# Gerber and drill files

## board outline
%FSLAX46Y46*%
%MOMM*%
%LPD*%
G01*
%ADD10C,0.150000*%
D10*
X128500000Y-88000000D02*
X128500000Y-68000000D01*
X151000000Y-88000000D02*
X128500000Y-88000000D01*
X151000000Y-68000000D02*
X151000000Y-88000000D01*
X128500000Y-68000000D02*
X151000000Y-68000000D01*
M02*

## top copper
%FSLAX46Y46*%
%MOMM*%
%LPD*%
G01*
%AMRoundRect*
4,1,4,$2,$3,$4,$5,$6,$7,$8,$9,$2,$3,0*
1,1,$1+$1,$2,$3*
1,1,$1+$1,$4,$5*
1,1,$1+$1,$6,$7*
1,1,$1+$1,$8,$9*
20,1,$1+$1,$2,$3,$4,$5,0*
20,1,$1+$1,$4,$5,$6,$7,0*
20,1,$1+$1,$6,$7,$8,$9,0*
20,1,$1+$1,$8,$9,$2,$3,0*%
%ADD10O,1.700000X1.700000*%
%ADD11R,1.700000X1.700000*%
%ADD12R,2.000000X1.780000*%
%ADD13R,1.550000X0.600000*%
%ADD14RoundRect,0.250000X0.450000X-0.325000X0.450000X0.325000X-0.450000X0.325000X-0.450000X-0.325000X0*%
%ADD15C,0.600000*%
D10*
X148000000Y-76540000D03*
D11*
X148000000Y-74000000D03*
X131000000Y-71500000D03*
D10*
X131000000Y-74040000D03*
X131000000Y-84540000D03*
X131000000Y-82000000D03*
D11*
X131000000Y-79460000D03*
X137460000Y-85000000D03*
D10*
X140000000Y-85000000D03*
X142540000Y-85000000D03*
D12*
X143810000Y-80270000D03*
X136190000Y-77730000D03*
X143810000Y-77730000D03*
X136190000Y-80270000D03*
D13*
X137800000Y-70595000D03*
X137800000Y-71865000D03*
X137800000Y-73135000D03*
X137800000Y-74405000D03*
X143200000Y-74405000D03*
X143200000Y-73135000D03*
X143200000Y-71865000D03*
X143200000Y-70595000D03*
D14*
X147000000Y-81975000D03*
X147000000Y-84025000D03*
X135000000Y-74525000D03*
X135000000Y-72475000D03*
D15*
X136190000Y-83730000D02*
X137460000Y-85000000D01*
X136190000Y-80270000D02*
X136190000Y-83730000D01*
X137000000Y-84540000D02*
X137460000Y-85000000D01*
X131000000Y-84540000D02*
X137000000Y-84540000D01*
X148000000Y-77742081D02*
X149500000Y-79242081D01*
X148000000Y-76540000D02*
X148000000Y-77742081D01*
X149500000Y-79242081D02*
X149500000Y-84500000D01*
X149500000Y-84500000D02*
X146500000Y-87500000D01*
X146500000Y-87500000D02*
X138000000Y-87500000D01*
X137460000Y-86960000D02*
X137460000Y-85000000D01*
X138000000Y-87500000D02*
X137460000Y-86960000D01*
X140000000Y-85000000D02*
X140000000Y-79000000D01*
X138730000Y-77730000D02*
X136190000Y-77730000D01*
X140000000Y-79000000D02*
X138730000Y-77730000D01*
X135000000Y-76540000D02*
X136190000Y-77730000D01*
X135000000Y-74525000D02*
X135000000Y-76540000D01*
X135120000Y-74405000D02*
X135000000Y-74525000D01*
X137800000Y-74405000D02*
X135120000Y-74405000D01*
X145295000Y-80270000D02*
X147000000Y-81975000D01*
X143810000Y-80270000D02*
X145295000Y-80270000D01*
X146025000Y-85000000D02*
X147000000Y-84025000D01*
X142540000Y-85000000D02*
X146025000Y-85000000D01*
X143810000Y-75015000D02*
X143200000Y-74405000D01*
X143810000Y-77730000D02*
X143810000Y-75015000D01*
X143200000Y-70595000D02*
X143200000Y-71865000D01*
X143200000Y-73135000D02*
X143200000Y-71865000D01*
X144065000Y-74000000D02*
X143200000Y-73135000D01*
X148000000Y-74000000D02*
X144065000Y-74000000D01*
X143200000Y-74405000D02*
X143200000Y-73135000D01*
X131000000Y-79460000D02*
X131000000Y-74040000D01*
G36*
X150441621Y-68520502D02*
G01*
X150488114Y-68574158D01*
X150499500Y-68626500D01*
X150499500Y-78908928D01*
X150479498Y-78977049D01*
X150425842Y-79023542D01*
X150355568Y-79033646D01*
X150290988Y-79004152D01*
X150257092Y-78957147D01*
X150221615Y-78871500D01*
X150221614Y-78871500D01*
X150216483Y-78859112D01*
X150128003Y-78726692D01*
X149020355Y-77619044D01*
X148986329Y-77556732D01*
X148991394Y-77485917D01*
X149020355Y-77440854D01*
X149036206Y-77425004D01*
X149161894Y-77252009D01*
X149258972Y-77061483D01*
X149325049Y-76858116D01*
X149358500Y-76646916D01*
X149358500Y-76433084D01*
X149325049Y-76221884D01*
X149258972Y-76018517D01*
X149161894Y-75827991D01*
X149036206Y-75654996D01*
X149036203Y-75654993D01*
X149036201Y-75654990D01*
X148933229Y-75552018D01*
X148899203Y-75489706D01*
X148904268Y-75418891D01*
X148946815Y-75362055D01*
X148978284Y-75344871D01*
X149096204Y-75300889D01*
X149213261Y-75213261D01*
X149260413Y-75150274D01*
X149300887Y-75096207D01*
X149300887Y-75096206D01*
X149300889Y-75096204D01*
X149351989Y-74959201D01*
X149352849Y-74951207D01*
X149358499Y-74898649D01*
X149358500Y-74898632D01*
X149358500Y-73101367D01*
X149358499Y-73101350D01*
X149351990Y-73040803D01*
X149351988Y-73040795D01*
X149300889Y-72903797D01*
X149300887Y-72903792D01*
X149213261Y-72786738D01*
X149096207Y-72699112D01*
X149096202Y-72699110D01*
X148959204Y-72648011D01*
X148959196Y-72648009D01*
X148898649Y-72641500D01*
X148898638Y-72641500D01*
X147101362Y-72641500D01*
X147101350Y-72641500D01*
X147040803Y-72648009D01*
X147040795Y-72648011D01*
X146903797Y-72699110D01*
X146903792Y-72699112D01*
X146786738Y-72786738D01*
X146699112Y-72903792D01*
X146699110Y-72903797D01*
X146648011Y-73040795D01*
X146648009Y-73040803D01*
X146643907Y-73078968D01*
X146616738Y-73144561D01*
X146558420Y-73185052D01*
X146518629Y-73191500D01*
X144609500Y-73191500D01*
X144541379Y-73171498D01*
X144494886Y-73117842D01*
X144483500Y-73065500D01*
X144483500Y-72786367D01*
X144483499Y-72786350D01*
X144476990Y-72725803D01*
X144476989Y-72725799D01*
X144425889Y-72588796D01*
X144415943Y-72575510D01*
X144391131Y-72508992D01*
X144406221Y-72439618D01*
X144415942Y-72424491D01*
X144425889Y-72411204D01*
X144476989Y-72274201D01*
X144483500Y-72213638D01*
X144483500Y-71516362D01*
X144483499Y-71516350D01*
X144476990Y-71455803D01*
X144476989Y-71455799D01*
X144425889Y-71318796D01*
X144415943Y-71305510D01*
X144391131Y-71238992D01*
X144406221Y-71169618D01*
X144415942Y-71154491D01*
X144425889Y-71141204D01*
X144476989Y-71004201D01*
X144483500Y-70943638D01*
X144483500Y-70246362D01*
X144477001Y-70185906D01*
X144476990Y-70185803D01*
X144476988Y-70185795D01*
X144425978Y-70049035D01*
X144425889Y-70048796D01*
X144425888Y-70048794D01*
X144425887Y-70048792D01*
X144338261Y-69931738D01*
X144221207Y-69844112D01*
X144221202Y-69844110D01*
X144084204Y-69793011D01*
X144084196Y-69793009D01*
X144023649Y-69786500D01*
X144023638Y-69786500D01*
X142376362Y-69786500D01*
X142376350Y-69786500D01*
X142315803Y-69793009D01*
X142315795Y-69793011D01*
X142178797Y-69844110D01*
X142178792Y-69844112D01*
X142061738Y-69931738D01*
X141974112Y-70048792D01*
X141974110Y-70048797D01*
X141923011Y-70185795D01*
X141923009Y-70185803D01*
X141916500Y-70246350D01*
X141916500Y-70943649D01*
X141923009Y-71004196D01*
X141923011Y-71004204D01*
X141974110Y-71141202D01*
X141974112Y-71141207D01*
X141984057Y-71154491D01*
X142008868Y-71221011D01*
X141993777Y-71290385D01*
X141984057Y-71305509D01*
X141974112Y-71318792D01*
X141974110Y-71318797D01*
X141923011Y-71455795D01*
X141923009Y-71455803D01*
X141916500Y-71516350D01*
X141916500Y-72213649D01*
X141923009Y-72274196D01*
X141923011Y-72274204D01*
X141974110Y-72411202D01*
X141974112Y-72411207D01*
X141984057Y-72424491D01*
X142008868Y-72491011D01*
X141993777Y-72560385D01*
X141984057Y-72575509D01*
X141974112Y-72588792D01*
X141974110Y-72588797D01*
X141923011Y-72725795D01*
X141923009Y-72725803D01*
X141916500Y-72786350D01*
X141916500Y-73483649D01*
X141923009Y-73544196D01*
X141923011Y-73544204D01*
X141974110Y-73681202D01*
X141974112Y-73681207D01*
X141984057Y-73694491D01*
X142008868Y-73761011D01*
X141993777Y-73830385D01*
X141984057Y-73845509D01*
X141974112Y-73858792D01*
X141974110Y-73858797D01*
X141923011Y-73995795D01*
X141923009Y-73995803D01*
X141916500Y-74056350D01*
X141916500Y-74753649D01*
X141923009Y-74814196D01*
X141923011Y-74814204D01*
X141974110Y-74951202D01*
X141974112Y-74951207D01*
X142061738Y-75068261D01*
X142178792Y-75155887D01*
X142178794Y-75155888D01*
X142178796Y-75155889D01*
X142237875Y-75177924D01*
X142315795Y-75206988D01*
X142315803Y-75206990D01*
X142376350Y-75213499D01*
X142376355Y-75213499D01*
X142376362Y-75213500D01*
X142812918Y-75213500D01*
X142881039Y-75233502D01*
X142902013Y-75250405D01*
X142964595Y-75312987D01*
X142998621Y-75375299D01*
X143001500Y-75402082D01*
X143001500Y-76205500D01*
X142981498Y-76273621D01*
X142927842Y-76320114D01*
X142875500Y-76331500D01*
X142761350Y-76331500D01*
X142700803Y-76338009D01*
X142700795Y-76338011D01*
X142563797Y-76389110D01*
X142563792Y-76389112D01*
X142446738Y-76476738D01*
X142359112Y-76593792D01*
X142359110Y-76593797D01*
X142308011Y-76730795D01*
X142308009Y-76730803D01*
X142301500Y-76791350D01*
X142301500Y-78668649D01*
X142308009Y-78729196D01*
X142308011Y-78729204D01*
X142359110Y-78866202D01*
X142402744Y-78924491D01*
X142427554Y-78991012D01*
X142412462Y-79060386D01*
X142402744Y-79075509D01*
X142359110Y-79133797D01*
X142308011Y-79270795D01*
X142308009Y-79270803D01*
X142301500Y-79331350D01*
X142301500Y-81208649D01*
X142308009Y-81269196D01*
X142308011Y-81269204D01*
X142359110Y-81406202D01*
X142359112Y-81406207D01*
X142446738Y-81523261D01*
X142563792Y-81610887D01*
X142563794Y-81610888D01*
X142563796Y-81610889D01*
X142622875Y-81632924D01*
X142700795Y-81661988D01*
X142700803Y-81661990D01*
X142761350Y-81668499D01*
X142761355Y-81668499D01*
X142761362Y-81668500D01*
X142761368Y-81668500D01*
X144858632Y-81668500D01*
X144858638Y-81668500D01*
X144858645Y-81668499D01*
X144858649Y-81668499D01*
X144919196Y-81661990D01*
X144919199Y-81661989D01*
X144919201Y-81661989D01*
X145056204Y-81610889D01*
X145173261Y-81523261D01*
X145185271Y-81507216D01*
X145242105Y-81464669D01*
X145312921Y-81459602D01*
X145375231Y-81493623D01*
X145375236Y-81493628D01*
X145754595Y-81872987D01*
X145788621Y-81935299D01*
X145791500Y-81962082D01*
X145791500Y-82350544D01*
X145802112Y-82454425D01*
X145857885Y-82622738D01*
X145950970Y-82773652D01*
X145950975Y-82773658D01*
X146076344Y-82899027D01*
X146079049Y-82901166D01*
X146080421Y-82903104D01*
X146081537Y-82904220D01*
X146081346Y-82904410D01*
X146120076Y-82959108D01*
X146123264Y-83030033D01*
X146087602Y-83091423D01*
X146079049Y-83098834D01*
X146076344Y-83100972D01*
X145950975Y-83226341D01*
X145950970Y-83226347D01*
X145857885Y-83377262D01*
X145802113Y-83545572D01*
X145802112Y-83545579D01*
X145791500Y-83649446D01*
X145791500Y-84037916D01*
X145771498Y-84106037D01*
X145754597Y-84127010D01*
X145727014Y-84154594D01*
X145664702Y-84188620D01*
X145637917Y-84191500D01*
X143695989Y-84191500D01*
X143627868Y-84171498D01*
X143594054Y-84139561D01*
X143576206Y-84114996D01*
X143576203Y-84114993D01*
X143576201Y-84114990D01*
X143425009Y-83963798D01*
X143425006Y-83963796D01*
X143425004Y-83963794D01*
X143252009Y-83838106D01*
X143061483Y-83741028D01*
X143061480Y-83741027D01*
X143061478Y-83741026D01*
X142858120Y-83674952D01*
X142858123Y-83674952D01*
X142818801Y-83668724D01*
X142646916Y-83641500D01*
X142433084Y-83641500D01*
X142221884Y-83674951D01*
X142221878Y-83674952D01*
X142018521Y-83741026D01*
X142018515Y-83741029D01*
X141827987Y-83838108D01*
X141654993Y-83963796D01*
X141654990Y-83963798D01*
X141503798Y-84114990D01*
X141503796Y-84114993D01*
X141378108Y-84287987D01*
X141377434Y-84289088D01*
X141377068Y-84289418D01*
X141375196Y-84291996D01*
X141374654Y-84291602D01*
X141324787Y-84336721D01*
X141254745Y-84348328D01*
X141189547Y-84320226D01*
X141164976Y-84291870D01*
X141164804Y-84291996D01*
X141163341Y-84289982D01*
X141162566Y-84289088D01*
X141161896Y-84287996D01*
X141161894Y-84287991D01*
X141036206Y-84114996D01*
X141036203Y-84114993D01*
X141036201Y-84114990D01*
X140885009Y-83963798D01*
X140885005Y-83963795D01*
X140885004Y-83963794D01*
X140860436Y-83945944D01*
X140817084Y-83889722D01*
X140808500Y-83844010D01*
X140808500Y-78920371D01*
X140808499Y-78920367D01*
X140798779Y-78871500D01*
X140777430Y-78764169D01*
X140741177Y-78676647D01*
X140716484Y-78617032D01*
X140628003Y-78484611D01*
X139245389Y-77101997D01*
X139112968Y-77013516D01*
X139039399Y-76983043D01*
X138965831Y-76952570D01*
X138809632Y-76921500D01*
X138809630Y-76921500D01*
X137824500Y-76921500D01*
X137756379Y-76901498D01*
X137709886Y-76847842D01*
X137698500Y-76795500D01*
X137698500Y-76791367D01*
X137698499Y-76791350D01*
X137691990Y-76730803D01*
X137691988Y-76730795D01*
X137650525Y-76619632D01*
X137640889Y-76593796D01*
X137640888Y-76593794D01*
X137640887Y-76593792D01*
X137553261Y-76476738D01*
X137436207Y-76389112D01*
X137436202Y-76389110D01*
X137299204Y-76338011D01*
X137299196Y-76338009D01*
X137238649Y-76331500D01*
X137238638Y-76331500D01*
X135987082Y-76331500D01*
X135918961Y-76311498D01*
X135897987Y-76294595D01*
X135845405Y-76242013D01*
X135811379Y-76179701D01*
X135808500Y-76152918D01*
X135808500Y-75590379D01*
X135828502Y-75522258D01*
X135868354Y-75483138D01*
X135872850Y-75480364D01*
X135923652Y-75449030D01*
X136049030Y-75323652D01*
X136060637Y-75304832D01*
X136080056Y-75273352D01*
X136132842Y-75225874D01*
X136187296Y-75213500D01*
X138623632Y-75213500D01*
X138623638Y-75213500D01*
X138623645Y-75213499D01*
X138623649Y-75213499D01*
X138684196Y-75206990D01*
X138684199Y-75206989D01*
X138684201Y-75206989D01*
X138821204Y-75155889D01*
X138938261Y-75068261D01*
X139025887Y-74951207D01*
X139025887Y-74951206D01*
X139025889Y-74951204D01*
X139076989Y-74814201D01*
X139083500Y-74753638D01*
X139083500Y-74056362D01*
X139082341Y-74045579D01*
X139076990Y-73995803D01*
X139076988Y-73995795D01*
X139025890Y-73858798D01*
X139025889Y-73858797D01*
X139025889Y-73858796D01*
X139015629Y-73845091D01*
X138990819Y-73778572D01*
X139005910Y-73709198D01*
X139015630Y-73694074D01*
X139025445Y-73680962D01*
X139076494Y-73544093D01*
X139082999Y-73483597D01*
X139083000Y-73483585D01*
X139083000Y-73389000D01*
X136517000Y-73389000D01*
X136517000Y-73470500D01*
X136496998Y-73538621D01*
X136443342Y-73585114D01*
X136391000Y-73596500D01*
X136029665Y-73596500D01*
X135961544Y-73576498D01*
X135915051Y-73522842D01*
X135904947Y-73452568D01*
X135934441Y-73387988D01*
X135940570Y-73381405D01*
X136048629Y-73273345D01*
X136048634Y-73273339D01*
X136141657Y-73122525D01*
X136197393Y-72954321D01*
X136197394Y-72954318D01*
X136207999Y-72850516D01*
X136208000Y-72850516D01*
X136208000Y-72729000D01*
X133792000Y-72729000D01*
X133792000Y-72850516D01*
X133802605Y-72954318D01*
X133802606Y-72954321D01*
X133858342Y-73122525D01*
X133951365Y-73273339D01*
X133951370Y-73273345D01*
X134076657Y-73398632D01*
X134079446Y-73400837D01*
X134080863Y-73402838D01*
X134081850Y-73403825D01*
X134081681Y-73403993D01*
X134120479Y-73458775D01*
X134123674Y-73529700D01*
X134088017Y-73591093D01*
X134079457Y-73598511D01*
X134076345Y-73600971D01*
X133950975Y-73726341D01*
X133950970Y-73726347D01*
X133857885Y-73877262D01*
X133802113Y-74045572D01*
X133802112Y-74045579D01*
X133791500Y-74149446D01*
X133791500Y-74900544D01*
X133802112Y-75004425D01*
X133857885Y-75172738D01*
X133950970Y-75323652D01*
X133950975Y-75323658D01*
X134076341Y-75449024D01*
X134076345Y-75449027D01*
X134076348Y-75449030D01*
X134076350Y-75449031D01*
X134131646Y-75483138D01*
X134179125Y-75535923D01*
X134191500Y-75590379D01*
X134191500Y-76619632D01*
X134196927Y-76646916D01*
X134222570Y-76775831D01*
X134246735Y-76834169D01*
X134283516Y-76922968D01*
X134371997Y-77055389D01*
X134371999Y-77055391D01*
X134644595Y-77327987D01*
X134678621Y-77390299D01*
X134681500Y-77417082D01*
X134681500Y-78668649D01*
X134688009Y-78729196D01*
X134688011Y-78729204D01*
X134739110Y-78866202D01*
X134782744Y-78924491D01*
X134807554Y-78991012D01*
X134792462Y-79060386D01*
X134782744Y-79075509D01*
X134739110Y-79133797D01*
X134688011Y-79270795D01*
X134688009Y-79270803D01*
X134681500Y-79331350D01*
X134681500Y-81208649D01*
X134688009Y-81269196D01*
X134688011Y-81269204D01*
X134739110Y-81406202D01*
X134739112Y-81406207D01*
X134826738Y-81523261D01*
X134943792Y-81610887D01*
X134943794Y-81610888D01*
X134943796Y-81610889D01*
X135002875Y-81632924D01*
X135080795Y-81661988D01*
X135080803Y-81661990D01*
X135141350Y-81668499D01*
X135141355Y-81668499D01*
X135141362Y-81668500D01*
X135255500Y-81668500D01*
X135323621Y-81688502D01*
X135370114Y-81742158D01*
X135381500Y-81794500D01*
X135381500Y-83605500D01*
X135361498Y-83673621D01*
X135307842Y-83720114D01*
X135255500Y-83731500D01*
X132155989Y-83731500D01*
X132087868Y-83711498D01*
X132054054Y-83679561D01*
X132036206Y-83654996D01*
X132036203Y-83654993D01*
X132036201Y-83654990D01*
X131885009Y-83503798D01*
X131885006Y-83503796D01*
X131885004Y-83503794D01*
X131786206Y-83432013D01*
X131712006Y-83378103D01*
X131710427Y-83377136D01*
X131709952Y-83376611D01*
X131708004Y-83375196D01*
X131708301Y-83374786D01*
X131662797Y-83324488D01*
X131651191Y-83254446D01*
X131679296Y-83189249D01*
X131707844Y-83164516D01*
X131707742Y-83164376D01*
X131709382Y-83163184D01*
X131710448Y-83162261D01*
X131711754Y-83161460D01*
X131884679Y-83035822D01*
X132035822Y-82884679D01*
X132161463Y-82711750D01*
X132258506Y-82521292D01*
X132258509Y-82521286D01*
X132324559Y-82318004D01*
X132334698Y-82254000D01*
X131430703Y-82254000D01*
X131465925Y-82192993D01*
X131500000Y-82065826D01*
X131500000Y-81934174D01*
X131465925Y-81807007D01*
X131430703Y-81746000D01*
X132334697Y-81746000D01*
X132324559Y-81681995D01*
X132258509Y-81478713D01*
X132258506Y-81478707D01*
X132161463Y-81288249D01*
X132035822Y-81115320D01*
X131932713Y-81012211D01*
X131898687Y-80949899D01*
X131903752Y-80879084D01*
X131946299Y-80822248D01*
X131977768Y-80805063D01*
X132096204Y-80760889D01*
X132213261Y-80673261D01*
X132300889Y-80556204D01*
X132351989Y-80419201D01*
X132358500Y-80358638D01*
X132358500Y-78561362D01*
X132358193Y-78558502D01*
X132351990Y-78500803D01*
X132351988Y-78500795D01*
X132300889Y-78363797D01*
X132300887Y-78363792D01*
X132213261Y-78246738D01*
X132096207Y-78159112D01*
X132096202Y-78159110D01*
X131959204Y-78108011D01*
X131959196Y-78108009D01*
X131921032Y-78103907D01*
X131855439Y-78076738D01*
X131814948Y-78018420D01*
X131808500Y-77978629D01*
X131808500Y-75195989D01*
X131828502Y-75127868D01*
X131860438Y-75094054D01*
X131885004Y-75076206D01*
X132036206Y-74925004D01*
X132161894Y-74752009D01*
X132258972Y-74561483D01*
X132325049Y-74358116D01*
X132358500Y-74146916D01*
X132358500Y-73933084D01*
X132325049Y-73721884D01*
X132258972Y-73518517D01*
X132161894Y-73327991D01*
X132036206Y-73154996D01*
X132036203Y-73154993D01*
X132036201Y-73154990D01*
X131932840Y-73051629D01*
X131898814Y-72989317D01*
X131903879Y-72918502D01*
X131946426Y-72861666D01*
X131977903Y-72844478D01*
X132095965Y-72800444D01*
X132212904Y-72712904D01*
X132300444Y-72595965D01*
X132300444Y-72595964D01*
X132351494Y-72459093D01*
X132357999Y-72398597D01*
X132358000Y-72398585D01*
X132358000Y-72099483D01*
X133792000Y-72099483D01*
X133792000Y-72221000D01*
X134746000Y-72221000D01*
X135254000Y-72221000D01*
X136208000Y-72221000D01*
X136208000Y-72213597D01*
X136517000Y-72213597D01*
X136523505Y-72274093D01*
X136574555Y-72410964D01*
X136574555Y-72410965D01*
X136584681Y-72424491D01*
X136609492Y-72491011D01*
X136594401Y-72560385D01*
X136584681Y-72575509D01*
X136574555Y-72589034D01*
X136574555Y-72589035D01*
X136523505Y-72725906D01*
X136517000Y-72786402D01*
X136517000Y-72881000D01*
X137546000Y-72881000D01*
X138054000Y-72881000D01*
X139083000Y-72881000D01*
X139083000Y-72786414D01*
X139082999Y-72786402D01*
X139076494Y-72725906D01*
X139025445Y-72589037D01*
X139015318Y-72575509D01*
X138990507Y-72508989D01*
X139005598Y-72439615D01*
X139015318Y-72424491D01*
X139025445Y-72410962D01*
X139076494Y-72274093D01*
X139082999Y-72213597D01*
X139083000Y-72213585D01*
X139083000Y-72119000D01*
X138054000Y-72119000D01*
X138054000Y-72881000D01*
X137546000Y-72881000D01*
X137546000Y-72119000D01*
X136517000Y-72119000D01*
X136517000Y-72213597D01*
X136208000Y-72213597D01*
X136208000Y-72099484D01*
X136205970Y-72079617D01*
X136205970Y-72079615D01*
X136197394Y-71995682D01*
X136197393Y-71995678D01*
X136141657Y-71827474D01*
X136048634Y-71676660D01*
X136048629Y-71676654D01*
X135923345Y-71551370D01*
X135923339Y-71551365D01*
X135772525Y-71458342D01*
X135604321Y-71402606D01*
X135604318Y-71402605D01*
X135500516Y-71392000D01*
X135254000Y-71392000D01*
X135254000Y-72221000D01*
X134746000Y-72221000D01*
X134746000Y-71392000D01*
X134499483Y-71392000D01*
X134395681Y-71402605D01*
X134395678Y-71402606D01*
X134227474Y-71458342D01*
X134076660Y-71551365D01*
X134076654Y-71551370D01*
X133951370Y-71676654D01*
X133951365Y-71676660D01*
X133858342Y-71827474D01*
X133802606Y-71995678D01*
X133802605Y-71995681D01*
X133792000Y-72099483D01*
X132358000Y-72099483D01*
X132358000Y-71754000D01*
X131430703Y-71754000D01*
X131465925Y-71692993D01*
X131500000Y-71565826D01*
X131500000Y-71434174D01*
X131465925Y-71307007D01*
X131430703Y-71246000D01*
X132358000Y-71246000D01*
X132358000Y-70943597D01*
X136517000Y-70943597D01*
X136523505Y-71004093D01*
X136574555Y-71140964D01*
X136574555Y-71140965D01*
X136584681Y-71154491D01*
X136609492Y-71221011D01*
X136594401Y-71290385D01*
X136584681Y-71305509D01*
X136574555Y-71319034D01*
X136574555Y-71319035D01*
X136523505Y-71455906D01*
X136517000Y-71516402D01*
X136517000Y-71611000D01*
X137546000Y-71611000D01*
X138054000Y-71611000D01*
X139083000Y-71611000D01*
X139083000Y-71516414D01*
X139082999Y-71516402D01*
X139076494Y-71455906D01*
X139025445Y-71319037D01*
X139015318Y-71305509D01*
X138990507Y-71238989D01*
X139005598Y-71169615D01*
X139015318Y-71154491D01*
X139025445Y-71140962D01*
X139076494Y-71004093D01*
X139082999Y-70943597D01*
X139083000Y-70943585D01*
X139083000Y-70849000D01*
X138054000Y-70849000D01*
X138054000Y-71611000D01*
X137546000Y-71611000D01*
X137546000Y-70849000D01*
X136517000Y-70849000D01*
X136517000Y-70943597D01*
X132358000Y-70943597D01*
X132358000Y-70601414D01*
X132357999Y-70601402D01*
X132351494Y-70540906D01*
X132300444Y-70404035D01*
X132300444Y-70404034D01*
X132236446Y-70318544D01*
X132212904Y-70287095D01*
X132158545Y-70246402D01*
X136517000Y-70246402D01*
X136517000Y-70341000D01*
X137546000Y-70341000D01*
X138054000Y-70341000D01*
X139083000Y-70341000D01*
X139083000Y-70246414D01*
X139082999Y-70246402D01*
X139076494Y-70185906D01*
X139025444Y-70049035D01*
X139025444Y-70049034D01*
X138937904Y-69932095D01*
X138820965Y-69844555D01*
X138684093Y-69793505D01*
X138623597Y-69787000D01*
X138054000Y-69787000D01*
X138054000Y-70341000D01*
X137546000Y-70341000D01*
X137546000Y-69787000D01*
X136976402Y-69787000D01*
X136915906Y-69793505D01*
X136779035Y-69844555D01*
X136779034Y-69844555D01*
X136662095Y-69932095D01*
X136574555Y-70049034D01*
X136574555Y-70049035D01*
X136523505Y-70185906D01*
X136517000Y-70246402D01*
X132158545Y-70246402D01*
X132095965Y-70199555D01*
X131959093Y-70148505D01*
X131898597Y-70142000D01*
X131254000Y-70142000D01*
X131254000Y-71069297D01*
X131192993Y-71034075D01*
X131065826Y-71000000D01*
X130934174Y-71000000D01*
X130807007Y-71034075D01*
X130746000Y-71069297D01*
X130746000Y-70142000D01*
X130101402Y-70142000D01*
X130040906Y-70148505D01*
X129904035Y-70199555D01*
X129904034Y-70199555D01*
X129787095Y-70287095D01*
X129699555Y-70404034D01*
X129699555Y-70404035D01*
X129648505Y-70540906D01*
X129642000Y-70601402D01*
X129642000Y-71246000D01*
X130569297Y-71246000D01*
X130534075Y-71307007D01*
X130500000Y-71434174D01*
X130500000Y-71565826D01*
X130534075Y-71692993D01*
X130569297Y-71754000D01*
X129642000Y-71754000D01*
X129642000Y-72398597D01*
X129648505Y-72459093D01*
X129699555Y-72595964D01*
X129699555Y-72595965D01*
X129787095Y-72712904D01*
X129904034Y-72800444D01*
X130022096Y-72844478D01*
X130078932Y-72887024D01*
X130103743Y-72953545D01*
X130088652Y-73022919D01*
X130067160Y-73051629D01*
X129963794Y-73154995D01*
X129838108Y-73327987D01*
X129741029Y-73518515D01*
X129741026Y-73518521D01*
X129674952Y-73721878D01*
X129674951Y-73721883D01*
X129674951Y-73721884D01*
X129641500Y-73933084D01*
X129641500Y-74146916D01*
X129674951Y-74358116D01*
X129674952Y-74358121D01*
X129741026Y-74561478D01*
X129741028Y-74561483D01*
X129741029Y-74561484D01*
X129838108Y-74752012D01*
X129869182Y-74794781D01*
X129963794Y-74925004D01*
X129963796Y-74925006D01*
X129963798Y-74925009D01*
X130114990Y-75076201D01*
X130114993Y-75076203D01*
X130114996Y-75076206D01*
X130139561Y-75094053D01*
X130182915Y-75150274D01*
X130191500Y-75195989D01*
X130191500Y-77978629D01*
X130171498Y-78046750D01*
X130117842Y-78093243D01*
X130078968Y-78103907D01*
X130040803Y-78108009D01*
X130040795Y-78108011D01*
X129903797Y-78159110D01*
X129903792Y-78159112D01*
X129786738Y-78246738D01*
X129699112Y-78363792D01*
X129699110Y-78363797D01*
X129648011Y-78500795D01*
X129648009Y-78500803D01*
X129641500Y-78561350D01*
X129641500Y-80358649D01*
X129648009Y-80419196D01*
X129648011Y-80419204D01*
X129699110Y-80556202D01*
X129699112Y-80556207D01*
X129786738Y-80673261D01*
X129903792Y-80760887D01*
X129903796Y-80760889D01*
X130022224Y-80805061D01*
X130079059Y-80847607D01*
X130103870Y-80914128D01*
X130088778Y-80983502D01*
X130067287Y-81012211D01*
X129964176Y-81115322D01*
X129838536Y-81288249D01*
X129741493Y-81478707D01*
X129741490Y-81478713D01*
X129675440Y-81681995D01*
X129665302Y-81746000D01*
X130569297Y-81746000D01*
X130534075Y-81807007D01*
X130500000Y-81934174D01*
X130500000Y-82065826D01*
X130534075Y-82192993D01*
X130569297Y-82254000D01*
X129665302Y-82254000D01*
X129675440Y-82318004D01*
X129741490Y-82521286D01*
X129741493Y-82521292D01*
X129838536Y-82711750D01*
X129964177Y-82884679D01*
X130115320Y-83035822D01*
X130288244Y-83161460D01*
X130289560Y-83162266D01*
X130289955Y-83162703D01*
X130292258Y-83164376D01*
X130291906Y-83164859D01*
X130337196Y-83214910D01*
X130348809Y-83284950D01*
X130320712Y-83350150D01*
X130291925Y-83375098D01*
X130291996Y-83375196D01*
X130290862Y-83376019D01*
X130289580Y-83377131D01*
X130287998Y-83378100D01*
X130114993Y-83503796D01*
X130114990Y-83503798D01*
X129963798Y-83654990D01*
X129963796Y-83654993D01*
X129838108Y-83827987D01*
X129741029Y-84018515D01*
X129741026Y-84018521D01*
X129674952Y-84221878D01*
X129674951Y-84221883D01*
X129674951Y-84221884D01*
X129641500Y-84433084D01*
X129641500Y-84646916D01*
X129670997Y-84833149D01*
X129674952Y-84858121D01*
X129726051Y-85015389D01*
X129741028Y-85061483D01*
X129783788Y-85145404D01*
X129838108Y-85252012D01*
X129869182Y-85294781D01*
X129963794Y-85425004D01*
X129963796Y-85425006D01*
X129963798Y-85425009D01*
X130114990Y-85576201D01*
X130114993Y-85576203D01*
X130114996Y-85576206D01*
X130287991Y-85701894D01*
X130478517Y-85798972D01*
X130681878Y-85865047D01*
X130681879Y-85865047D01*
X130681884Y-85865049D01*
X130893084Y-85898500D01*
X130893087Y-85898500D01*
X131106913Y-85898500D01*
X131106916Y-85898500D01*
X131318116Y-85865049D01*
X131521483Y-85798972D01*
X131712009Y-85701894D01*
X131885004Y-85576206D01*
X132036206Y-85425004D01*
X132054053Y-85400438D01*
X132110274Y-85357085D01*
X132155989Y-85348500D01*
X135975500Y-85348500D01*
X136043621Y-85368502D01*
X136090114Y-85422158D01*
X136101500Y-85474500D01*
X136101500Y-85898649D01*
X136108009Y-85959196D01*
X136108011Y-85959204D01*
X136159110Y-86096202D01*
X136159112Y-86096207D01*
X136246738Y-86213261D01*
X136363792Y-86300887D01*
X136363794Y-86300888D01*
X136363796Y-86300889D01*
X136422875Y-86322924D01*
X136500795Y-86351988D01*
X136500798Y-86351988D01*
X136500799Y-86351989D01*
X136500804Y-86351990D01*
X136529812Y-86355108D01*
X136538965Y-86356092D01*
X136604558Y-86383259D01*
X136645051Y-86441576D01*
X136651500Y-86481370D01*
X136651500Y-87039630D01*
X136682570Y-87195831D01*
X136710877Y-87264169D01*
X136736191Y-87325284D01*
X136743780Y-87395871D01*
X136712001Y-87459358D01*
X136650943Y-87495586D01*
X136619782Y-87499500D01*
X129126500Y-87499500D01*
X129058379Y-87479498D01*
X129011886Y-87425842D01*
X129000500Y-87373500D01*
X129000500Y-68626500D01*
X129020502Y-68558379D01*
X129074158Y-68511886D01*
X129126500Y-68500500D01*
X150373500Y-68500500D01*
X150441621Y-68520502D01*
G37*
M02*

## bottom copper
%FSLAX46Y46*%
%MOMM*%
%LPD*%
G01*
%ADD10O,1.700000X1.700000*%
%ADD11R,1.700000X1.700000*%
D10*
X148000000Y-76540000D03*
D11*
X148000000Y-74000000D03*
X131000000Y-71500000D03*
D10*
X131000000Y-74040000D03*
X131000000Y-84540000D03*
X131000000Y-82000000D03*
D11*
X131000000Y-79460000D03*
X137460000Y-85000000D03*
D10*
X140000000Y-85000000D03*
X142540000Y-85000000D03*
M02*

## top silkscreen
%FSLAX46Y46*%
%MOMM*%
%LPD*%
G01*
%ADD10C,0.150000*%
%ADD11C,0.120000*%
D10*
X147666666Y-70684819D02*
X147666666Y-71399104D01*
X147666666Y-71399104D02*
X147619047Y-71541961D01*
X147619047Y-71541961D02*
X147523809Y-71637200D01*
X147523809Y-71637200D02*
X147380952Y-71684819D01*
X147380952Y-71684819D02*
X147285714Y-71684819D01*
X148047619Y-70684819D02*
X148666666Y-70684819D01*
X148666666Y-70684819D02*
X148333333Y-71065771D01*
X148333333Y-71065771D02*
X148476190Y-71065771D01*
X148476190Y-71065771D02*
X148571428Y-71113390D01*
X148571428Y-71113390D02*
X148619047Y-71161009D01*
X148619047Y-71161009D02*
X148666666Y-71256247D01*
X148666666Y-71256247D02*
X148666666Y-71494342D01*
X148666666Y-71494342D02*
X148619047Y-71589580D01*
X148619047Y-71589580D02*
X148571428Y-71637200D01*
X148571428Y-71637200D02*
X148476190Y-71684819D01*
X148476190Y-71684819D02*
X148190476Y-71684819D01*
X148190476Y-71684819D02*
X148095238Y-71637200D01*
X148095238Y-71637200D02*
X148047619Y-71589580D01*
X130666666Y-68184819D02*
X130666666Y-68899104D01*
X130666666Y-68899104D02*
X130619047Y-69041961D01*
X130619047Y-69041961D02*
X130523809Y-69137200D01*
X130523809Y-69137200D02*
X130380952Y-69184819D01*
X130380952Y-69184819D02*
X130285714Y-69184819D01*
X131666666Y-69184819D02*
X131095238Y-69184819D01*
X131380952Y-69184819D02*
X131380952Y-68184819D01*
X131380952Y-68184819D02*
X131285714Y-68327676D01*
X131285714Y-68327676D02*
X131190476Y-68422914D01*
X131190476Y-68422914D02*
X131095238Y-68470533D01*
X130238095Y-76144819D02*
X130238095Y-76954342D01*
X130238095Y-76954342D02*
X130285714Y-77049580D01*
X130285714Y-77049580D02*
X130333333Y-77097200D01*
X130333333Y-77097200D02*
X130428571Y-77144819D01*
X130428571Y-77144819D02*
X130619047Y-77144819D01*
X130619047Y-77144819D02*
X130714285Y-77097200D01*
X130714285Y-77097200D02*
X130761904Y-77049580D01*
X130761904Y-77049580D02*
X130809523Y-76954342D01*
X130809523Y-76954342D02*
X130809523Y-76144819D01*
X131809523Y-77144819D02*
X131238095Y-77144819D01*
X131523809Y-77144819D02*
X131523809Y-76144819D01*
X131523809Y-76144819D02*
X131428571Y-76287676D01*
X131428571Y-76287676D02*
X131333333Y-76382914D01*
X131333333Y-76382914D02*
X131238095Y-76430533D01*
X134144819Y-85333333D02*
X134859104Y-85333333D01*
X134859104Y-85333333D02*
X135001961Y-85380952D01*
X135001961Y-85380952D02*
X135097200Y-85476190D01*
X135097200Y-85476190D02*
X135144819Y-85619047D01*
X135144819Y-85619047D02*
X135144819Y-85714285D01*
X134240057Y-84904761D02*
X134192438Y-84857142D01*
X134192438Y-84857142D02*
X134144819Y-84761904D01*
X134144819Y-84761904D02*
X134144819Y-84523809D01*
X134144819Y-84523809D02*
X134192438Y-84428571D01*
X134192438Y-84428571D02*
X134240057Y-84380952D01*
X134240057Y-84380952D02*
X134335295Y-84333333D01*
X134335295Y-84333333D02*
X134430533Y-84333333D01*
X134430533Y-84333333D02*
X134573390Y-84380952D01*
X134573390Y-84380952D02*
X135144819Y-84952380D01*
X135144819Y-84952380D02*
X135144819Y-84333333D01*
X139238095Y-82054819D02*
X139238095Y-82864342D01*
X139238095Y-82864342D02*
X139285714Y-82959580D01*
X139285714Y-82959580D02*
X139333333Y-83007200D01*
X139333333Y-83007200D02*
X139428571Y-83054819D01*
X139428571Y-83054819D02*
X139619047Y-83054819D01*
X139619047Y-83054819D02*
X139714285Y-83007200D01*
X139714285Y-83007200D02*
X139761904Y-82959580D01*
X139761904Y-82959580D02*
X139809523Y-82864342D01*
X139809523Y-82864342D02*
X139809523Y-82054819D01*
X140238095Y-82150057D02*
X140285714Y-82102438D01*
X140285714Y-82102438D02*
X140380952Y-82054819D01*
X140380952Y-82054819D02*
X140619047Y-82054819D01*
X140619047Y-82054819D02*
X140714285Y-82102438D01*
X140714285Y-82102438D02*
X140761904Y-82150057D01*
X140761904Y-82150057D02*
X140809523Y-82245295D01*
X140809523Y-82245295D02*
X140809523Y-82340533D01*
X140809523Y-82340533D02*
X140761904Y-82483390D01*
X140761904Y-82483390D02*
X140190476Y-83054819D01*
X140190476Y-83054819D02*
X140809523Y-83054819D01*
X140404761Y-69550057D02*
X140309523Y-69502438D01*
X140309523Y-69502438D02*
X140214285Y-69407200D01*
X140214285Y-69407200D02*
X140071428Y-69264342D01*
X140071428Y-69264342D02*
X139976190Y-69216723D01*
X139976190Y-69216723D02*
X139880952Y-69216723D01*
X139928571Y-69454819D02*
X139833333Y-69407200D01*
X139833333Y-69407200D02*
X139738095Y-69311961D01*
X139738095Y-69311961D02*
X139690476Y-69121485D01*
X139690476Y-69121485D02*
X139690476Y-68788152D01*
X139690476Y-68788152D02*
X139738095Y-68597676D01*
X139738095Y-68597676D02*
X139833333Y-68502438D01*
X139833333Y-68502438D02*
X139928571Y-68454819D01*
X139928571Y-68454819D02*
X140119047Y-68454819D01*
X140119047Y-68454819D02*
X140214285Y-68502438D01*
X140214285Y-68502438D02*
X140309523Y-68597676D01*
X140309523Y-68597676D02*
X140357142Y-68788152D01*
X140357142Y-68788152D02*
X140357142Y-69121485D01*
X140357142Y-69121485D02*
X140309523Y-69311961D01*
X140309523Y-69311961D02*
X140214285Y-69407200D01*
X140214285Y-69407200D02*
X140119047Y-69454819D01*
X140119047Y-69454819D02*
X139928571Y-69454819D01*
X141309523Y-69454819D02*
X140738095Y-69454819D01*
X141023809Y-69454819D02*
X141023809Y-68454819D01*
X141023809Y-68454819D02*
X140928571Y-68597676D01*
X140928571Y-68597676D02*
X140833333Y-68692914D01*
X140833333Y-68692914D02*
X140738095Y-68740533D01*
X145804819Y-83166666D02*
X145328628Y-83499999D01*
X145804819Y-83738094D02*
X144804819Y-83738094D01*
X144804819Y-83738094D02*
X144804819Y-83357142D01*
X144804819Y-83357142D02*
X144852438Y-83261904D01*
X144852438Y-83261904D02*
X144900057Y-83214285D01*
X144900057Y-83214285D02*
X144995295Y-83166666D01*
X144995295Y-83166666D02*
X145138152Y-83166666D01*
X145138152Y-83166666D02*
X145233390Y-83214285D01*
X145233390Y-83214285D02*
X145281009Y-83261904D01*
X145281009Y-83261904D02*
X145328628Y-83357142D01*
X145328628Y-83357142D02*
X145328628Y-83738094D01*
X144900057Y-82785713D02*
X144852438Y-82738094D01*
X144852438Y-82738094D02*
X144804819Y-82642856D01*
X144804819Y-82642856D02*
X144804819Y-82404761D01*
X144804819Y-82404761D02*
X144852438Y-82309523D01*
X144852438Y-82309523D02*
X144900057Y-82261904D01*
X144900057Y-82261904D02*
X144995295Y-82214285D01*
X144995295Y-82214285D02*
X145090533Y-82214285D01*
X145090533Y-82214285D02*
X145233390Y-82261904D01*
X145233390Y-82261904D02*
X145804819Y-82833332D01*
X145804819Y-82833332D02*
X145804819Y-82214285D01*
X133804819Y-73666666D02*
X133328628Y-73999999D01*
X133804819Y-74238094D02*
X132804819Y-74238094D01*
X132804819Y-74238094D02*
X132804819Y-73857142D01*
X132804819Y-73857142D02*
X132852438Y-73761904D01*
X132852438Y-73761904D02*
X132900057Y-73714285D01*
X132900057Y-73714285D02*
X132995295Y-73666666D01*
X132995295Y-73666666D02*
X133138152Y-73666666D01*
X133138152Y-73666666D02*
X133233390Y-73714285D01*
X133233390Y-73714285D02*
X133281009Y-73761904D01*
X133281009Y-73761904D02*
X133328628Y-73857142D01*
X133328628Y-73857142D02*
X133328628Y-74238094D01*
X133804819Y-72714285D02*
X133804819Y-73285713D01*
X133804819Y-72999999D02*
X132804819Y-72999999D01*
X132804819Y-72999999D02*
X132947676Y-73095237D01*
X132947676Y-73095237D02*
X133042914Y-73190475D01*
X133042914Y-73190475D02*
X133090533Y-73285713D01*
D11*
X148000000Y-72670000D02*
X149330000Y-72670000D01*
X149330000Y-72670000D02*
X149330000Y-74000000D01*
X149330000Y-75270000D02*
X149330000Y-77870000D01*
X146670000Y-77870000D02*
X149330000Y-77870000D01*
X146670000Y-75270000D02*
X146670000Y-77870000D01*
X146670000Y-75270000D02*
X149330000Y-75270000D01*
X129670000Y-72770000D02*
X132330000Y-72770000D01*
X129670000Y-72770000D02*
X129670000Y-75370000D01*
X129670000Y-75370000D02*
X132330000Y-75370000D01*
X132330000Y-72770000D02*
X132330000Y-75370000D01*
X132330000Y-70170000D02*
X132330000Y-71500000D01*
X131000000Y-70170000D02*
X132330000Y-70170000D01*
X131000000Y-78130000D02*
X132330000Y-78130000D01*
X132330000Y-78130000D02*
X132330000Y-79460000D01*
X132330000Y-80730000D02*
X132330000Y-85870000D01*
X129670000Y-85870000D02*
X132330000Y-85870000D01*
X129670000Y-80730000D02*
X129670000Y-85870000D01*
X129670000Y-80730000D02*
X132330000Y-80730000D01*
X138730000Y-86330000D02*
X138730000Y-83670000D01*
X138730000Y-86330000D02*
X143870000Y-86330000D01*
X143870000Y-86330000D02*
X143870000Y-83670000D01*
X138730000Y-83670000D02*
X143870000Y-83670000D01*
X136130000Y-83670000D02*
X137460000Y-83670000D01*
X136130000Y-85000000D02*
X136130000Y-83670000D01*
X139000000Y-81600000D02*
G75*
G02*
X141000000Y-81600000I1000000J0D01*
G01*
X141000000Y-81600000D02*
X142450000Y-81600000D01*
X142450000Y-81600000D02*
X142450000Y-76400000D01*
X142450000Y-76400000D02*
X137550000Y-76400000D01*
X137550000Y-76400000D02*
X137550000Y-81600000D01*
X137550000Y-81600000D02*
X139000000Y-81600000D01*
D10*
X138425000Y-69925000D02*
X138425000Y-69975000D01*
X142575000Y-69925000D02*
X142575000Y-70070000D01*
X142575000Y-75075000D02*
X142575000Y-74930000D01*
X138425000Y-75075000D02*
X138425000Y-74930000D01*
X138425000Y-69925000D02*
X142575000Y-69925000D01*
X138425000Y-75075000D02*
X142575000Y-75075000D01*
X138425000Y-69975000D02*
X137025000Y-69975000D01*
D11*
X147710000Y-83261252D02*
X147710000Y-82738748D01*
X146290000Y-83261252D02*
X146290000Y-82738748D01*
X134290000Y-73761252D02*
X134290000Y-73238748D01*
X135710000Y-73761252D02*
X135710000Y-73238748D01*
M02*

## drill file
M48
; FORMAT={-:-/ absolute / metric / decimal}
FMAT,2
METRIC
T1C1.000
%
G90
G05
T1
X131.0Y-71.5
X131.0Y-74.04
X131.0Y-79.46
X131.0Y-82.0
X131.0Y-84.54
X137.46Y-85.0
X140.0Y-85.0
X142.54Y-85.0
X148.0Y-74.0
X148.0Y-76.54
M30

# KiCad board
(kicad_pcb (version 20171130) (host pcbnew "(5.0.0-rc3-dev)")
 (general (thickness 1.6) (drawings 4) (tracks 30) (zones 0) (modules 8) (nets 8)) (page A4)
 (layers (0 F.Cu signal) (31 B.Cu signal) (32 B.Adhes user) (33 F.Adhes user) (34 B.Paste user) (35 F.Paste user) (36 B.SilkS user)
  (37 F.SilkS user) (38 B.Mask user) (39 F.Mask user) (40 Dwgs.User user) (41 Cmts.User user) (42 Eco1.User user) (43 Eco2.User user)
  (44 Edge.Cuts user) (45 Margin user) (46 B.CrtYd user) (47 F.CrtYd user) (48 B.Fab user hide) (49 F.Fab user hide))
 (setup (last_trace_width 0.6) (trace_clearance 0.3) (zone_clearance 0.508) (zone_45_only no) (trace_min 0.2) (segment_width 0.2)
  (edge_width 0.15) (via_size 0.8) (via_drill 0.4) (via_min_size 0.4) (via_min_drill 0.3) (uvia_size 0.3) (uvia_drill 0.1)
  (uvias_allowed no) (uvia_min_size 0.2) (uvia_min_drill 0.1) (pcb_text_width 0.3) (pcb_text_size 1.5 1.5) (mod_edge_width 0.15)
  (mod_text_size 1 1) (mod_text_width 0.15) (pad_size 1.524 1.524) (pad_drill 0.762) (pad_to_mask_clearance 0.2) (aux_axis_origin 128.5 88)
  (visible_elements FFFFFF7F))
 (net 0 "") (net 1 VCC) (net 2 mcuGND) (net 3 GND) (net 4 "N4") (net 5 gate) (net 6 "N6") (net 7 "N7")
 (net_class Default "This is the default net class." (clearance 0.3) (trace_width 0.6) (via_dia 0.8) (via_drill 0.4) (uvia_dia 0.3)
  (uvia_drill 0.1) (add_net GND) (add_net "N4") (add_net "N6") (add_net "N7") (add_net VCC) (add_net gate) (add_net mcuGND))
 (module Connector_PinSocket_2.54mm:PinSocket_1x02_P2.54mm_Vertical (layer F.Cu) (at 148 74)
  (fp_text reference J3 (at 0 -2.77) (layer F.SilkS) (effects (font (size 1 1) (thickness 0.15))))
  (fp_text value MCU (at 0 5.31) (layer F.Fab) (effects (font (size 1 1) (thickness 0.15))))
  (fp_line (start 0 -1.33) (end 1.33 -1.33) (layer F.SilkS) (width 0.12))
  (fp_line (start 1.33 -1.33) (end 1.33 0) (layer F.SilkS) (width 0.12))
  (fp_line (start 1.33 1.27) (end 1.33 3.87) (layer F.SilkS) (width 0.12))
  (fp_line (start -1.33 3.87) (end 1.33 3.87) (layer F.SilkS) (width 0.12))
  (fp_line (start -1.33 1.27) (end -1.33 3.87) (layer F.SilkS) (width 0.12))
  (fp_line (start -1.33 1.27) (end 1.33 1.27) (layer F.SilkS) (width 0.12))
  (pad 2 thru_hole oval (at 0 2.54) (size 1.7 1.7) (drill 1) (layers *.Cu *.Mask) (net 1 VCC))
  (pad 1 thru_hole rect (at 0 0) (size 1.7 1.7) (drill 1) (layers *.Cu *.Mask) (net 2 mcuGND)))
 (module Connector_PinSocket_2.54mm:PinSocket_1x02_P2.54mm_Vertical (layer F.Cu) (at 131 71.5)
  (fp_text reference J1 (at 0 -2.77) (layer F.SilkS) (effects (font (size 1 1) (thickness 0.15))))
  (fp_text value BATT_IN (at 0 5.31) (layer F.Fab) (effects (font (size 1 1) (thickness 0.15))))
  (fp_line (start -1.33 1.27) (end 1.33 1.27) (layer F.SilkS) (width 0.12))
  (fp_line (start -1.33 1.27) (end -1.33 3.87) (layer F.SilkS) (width 0.12))
  (fp_line (start -1.33 3.87) (end 1.33 3.87) (layer F.SilkS) (width 0.12))
  (fp_line (start 1.33 1.27) (end 1.33 3.87) (layer F.SilkS) (width 0.12))
  (fp_line (start 1.33 -1.33) (end 1.33 0) (layer F.SilkS) (width 0.12))
  (fp_line (start 0 -1.33) (end 1.33 -1.33) (layer F.SilkS) (width 0.12))
  (pad 1 thru_hole rect (at 0 0) (size 1.7 1.7) (drill 1) (layers *.Cu *.Mask) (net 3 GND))
  (pad 2 thru_hole oval (at 0 2.54) (size 1.7 1.7) (drill 1) (layers *.Cu *.Mask) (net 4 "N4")))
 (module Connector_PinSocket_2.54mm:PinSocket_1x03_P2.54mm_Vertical (layer F.Cu) (at 131 79.46)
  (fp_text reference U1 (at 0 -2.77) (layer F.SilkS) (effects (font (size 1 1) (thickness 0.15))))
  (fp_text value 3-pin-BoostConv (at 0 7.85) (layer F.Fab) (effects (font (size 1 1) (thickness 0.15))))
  (fp_line (start 0 -1.33) (end 1.33 -1.33) (layer F.SilkS) (width 0.12))
  (fp_line (start 1.33 -1.33) (end 1.33 0) (layer F.SilkS) (width 0.12))
  (fp_line (start 1.33 1.27) (end 1.33 6.41) (layer F.SilkS) (width 0.12))
  (fp_line (start -1.33 6.41) (end 1.33 6.41) (layer F.SilkS) (width 0.12))
  (fp_line (start -1.33 1.27) (end -1.33 6.41) (layer F.SilkS) (width 0.12))
  (fp_line (start -1.33 1.27) (end 1.33 1.27) (layer F.SilkS) (width 0.12))
  (pad 3 thru_hole oval (at 0 5.08) (size 1.7 1.7) (drill 1) (layers *.Cu *.Mask) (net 1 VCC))
  (pad 2 thru_hole oval (at 0 2.54) (size 1.7 1.7) (drill 1) (layers *.Cu *.Mask) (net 3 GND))
  (pad 1 thru_hole rect (at 0 0) (size 1.7 1.7) (drill 1) (layers *.Cu *.Mask) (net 4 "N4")))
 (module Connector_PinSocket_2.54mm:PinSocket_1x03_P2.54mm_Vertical (layer F.Cu) (at 137.46 85 90)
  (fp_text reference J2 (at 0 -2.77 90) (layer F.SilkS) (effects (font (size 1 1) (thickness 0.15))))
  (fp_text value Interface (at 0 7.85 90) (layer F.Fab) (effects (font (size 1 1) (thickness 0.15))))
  (fp_line (start -1.33 1.27) (end 1.33 1.27) (layer F.SilkS) (width 0.12))
  (fp_line (start -1.33 1.27) (end -1.33 6.41) (layer F.SilkS) (width 0.12))
  (fp_line (start -1.33 6.41) (end 1.33 6.41) (layer F.SilkS) (width 0.12))
  (fp_line (start 1.33 1.27) (end 1.33 6.41) (layer F.SilkS) (width 0.12))
  (fp_line (start 1.33 -1.33) (end 1.33 0) (layer F.SilkS) (width 0.12))
  (fp_line (start 0 -1.33) (end 1.33 -1.33) (layer F.SilkS) (width 0.12))
  (pad 1 thru_hole rect (at 0 0 90) (size 1.7 1.7) (drill 1) (layers *.Cu *.Mask) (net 1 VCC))
  (pad 2 thru_hole oval (at 0 2.54 90) (size 1.7 1.7) (drill 1) (layers *.Cu *.Mask) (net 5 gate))
  (pad 3 thru_hole oval (at 0 5.08 90) (size 1.7 1.7) (drill 1) (layers *.Cu *.Mask) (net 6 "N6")))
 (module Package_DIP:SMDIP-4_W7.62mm (layer F.Cu) (at 140 79 180)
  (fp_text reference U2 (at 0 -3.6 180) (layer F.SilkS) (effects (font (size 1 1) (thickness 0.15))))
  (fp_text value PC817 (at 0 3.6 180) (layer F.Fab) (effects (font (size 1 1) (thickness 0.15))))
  (fp_arc (start 0 -2.6) (end -1 -2.6) (angle -180) (layer F.SilkS) (width 0.12))
  (fp_line (start -1 -2.6) (end -2.45 -2.6) (layer F.SilkS) (width 0.12))
  (fp_line (start -2.45 -2.6) (end -2.45 2.6) (layer F.SilkS) (width 0.12))
  (fp_line (start -2.45 2.6) (end 2.45 2.6) (layer F.SilkS) (width 0.12))
  (fp_line (start 2.45 2.6) (end 2.45 -2.6) (layer F.SilkS) (width 0.12))
  (fp_line (start 2.45 -2.6) (end 1 -2.6) (layer F.SilkS) (width 0.12))
  (pad 1 smd rect (at -3.81 -1.27 180) (size 2 1.78) (layers F.Cu F.Paste F.Mask) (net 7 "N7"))
  (pad 3 smd rect (at 3.81 1.27 180) (size 2 1.78) (layers F.Cu F.Paste F.Mask) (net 5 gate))
  (pad 2 smd rect (at -3.81 1.27 180) (size 2 1.78) (layers F.Cu F.Paste F.Mask) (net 2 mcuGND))
  (pad 4 smd rect (at 3.81 -1.27 180) (size 2 1.78) (layers F.Cu F.Paste F.Mask) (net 1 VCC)))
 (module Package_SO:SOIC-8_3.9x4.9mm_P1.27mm (layer F.Cu) (at 140.5 72.5)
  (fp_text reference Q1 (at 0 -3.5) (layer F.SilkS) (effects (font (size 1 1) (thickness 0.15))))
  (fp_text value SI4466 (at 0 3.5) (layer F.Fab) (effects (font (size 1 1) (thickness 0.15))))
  (fp_line (start -2.075 -2.575) (end -2.075 -2.525) (layer F.SilkS) (width 0.15))
  (fp_line (start 2.075 -2.575) (end 2.075 -2.43) (layer F.SilkS) (width 0.15))
  (fp_line (start 2.075 2.575) (end 2.075 2.43) (layer F.SilkS) (width 0.15))
  (fp_line (start -2.075 2.575) (end -2.075 2.43) (layer F.SilkS) (width 0.15))
  (fp_line (start -2.075 -2.575) (end 2.075 -2.575) (layer F.SilkS) (width 0.15))
  (fp_line (start -2.075 2.575) (end 2.075 2.575) (layer F.SilkS) (width 0.15))
  (fp_line (start -2.075 -2.525) (end -3.475 -2.525) (layer F.SilkS) (width 0.15))
  (pad 1 smd rect (at -2.7 -1.905) (size 1.55 0.6) (layers F.Cu F.Paste F.Mask) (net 3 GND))
  (pad 2 smd rect (at -2.7 -0.635) (size 1.55 0.6) (layers F.Cu F.Paste F.Mask) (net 3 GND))
  (pad 3 smd rect (at -2.7 0.635) (size 1.55 0.6) (layers F.Cu F.Paste F.Mask) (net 3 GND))
  (pad 4 smd rect (at -2.7 1.905) (size 1.55 0.6) (layers F.Cu F.Paste F.Mask) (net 5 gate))
  (pad 5 smd rect (at 2.7 1.905) (size 1.55 0.6) (layers F.Cu F.Paste F.Mask) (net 2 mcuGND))
  (pad 6 smd rect (at 2.7 0.635) (size 1.55 0.6) (layers F.Cu F.Paste F.Mask) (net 2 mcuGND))
  (pad 7 smd rect (at 2.7 -0.635) (size 1.55 0.6) (layers F.Cu F.Paste F.Mask) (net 2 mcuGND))
  (pad 8 smd rect (at 2.7 -1.905) (size 1.55 0.6) (layers F.Cu F.Paste F.Mask) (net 2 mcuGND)))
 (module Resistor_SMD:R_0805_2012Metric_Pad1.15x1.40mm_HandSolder (layer F.Cu) (at 147 83 90)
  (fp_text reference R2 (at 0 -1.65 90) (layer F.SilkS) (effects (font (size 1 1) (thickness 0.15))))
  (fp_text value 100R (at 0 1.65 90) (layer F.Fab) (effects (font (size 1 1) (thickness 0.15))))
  (fp_line (start -0.261252 0.71) (end 0.261252 0.71) (layer F.SilkS) (width 0.12))
  (fp_line (start -0.261252 -0.71) (end 0.261252 -0.71) (layer F.SilkS) (width 0.12))
  (pad 2 smd roundrect (at 1.025 0 90) (size 1.15 1.4) (layers F.Cu F.Paste F.Mask) (roundrect_rratio 0.217391) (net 7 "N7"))
  (pad 1 smd roundrect (at -1.025 0 90) (size 1.15 1.4) (layers F.Cu F.Paste F.Mask) (roundrect_rratio 0.217391) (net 6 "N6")))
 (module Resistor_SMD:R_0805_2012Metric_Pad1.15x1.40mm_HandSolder (layer F.Cu) (at 135 73.5 90)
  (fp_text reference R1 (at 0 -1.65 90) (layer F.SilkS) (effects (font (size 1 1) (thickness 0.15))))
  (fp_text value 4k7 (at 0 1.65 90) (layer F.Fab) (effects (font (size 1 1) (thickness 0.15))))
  (fp_line (start -0.261252 -0.71) (end 0.261252 -0.71) (layer F.SilkS) (width 0.12))
  (fp_line (start -0.261252 0.71) (end 0.261252 0.71) (layer F.SilkS) (width 0.12))
  (pad 1 smd roundrect (at -1.025 0 90) (size 1.15 1.4) (layers F.Cu F.Paste F.Mask) (roundrect_rratio 0.217391) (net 5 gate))
  (pad 2 smd roundrect (at 1.025 0 90) (size 1.15 1.4) (layers F.Cu F.Paste F.Mask) (roundrect_rratio 0.217391) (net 3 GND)))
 (gr_line (start 128.5 88) (end 128.5 68) (layer Edge.Cuts) (width 0.15))
 (gr_line (start 151 88) (end 128.5 88) (layer Edge.Cuts) (width 0.15))
 (gr_line (start 151 68) (end 151 88) (layer Edge.Cuts) (width 0.15))
 (gr_line (start 128.5 68) (end 151 68) (layer Edge.Cuts) (width 0.15))
 (segment (start 136.19 83.73) (end 137.46 85) (width 0.6) (layer F.Cu) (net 1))
 (segment (start 136.19 80.27) (end 136.19 83.73) (width 0.6) (layer F.Cu) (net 1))
 (segment (start 137 84.54) (end 137.46 85) (width 0.6) (layer F.Cu) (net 1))
 (segment (start 131 84.54) (end 137 84.54) (width 0.6) (layer F.Cu) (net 1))
 (segment (start 148 77.742081) (end 149.5 79.242081) (width 0.6) (layer F.Cu) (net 1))
 (segment (start 148 76.54) (end 148 77.742081) (width 0.6) (layer F.Cu) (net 1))
 (segment (start 149.5 79.242081) (end 149.5 84.5) (width 0.6) (layer F.Cu) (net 1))
 (segment (start 149.5 84.5) (end 146.5 87.5) (width 0.6) (layer F.Cu) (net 1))
 (segment (start 146.5 87.5) (end 138 87.5) (width 0.6) (layer F.Cu) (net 1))
 (segment (start 137.46 86.96) (end 137.46 85) (width 0.6) (layer F.Cu) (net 1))
 (segment (start 138 87.5) (end 137.46 86.96) (width 0.6) (layer F.Cu) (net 1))
 (segment (start 140 85) (end 140 79) (width 0.6) (layer F.Cu) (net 5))
 (segment (start 138.73 77.73) (end 136.19 77.73) (width 0.6) (layer F.Cu) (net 5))
 (segment (start 140 79) (end 138.73 77.73) (width 0.6) (layer F.Cu) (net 5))
 (segment (start 135 76.54) (end 136.19 77.73) (width 0.6) (layer F.Cu) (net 5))
 (segment (start 135 74.525) (end 135 76.54) (width 0.6) (layer F.Cu) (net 5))
 (segment (start 135.12 74.405) (end 135 74.525) (width 0.6) (layer F.Cu) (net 5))
 (segment (start 137.8 74.405) (end 135.12 74.405) (width 0.6) (layer F.Cu) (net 5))
 (segment (start 145.295 80.27) (end 147 81.975) (width 0.6) (layer F.Cu) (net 7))
 (segment (start 143.81 80.27) (end 145.295 80.27) (width 0.6) (layer F.Cu) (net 7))
 (segment (start 146.025 85) (end 147 84.025) (width 0.6) (layer F.Cu) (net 6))
 (segment (start 142.54 85) (end 146.025 85) (width 0.6) (layer F.Cu) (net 6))
 (segment (start 143.81 75.015) (end 143.2 74.405) (width 0.6) (layer F.Cu) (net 2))
 (segment (start 143.81 77.73) (end 143.81 75.015) (width 0.6) (layer F.Cu) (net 2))
 (segment (start 143.2 70.595) (end 143.2 71.865) (width 0.6) (layer F.Cu) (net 2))
 (segment (start 143.2 73.135) (end 143.2 71.865) (width 0.6) (layer F.Cu) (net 2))
 (segment (start 144.065 74) (end 143.2 73.135) (width 0.6) (layer F.Cu) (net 2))
 (segment (start 148 74) (end 144.065 74) (width 0.6) (layer F.Cu) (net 2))
 (segment (start 143.2 74.405) (end 143.2 73.135) (width 0.6) (layer F.Cu) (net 2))
 (segment (start 131 79.46) (end 131 74.04) (width 0.6) (layer F.Cu) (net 4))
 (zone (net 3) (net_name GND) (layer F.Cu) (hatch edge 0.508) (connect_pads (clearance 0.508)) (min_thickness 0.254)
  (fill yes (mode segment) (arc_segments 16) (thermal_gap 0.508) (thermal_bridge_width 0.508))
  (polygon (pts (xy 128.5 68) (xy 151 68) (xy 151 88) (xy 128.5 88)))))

